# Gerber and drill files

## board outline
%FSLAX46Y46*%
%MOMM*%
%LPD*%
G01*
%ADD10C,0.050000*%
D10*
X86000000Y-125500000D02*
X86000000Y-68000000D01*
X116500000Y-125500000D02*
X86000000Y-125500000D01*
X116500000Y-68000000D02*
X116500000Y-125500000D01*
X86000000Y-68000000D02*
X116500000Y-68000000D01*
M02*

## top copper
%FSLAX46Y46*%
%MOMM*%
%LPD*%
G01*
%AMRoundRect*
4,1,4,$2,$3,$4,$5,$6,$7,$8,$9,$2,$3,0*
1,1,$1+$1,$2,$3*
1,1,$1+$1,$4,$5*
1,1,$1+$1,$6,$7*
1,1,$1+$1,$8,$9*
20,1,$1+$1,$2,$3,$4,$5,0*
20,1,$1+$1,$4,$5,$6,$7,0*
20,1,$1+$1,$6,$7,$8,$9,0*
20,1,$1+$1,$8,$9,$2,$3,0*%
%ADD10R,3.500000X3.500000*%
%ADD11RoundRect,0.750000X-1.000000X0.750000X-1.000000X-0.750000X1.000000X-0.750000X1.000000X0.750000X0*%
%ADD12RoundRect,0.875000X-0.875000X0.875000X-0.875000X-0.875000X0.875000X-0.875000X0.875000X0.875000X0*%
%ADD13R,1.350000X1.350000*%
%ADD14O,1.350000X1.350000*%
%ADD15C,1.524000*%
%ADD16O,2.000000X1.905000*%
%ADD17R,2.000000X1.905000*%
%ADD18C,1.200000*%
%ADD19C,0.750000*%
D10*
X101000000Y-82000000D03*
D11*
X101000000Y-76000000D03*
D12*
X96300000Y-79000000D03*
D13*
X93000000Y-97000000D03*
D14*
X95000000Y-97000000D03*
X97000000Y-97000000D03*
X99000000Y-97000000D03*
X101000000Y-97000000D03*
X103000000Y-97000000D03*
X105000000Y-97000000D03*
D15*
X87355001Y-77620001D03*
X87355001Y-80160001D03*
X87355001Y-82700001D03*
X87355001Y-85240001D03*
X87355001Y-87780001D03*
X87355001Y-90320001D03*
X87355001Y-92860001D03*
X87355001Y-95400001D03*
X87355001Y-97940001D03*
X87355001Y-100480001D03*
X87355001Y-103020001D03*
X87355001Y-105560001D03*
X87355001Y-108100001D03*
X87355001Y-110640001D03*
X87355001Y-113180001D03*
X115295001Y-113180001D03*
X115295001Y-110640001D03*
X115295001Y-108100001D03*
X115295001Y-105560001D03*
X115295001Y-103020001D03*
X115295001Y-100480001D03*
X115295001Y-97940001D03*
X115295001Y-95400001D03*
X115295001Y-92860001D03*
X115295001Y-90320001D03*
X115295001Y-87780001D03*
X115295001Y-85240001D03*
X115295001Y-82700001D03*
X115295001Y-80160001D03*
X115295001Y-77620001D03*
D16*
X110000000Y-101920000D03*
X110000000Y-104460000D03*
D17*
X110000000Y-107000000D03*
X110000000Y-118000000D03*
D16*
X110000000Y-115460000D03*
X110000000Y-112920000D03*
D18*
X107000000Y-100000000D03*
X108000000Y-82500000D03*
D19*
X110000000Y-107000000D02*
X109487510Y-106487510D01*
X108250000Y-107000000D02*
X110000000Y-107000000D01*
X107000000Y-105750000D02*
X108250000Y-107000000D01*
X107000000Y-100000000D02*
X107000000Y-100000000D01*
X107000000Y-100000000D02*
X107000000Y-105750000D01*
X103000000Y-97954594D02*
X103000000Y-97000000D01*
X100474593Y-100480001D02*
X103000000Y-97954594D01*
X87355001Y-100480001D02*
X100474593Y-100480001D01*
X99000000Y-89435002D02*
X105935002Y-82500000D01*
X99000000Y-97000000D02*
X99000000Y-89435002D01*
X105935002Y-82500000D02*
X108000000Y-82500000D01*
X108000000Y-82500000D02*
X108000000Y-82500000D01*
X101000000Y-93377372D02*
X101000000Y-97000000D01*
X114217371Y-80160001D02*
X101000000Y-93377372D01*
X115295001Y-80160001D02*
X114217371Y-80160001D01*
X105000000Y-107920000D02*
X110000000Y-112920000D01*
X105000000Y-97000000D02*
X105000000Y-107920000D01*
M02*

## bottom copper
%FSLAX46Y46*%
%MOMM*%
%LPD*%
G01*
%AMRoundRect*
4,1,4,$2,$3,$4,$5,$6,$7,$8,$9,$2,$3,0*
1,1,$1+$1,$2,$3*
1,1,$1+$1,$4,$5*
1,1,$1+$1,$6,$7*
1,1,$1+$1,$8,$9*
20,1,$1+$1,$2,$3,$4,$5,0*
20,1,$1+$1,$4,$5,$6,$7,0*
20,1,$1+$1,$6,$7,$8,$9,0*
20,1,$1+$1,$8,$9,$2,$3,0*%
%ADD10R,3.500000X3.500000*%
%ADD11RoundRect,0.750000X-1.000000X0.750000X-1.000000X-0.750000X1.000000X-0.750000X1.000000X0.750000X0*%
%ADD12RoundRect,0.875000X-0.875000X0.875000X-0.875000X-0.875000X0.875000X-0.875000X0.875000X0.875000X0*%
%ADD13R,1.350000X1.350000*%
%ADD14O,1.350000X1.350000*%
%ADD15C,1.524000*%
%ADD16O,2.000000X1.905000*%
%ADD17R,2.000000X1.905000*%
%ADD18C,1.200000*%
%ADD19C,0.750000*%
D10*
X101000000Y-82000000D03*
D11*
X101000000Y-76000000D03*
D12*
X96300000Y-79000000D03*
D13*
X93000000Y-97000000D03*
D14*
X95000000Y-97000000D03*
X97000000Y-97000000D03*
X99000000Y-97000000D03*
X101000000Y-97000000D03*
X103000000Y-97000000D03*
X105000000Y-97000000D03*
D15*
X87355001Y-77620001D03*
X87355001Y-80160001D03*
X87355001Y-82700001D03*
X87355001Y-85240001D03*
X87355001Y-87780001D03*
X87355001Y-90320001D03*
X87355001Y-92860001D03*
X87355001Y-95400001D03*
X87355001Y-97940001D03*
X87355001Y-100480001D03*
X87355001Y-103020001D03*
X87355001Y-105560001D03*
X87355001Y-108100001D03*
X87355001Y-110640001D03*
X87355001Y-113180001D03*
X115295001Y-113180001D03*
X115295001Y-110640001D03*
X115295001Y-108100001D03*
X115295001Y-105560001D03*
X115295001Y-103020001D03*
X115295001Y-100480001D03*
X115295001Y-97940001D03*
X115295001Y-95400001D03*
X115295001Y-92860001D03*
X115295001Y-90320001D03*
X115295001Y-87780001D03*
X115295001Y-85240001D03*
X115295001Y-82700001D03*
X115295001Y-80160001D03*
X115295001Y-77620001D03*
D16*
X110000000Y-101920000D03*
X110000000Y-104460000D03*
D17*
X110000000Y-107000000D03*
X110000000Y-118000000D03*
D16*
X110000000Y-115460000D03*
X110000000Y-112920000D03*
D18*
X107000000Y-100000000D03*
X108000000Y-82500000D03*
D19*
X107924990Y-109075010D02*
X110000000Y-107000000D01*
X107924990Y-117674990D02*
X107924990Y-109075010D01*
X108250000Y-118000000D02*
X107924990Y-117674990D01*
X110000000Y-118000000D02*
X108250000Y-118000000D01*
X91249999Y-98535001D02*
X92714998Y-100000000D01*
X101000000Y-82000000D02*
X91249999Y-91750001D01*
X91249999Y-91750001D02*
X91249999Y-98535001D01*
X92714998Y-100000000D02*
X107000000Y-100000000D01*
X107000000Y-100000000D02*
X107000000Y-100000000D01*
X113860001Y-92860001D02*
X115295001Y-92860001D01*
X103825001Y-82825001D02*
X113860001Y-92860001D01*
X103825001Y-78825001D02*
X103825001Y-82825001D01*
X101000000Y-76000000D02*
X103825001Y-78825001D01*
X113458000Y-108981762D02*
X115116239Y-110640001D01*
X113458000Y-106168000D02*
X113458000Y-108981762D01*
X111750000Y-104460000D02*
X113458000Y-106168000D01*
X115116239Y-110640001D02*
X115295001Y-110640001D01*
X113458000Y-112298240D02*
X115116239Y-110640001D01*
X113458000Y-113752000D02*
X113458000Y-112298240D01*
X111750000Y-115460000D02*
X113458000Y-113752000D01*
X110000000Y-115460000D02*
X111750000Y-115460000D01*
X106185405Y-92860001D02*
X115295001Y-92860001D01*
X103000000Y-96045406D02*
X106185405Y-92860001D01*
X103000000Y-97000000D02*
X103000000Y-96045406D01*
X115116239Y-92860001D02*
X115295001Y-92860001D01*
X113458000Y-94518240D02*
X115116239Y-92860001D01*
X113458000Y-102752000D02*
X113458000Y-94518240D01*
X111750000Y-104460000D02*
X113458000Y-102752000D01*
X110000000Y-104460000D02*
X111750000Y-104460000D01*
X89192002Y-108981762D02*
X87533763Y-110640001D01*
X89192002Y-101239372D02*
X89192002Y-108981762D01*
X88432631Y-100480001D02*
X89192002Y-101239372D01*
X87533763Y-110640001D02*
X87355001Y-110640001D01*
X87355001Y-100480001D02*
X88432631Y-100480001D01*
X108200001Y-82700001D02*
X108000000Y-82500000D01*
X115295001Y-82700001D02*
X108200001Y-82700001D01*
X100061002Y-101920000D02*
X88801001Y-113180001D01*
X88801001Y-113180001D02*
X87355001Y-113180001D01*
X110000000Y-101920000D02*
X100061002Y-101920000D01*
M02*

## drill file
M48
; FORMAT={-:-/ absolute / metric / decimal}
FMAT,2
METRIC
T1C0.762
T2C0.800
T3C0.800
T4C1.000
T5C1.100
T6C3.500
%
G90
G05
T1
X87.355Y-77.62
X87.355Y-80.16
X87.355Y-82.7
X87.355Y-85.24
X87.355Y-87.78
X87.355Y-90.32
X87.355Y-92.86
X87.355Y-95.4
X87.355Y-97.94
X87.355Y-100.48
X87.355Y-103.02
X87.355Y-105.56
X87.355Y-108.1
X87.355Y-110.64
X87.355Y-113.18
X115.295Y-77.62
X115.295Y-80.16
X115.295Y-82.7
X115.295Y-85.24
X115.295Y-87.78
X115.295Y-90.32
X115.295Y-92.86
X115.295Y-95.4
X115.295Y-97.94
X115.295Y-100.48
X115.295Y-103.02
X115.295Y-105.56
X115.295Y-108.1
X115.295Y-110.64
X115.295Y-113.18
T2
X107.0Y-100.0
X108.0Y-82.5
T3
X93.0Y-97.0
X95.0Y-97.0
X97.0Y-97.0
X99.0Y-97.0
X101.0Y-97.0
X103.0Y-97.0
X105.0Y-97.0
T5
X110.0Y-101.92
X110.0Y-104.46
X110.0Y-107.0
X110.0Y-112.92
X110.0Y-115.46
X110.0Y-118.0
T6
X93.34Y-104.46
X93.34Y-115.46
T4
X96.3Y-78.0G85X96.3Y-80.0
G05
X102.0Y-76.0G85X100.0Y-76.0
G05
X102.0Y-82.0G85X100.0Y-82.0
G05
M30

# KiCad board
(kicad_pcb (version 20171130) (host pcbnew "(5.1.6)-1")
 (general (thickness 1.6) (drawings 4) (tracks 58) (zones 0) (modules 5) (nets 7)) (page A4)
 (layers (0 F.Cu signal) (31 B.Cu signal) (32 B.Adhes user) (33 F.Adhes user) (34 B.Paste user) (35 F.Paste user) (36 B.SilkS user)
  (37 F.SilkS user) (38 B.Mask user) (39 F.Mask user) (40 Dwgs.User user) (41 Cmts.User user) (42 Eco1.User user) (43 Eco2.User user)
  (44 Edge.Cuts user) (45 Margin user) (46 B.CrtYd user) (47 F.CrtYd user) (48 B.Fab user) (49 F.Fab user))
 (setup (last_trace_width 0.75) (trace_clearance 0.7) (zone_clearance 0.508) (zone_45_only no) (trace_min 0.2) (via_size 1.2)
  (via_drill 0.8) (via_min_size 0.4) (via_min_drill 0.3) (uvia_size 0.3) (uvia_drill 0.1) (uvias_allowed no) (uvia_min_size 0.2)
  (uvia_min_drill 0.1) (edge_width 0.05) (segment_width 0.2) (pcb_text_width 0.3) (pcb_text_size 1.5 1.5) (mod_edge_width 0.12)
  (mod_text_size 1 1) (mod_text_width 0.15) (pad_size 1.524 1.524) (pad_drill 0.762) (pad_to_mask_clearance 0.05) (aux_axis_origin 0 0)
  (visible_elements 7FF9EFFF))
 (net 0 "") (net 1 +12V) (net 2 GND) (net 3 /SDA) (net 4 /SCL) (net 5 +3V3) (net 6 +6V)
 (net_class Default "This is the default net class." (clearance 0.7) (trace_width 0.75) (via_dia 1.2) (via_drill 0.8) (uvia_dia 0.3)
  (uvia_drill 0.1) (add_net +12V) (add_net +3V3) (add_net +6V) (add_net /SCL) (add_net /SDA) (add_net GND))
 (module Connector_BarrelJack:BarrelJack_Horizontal (layer F.Cu) (at 101 82 270)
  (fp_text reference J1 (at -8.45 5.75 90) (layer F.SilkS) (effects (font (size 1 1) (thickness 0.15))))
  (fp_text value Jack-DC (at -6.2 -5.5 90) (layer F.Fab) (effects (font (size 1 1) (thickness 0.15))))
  (pad 1 thru_hole rect (at 0 0 270) (size 3.5 3.5) (drill oval 1 3) (layers *.Cu *.Mask) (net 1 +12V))
  (pad 2 thru_hole roundrect (at -6 0 270) (size 3 3.5) (drill oval 1 3) (layers *.Cu *.Mask) (roundrect_rratio 0.25) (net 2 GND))
  (pad 3 thru_hole roundrect (at -3 4.7 270) (size 3.5 3.5) (drill oval 3 1) (layers *.Cu *.Mask) (roundrect_rratio 0.25)))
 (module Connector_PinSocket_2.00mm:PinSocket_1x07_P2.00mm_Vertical (layer F.Cu) (at 93 97 90)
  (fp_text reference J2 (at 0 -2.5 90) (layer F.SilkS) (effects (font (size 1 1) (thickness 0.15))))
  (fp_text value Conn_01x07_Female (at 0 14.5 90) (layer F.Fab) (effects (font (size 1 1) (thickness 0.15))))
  (pad 1 thru_hole rect (at 0 0 90) (size 1.35 1.35) (drill 0.8) (layers *.Cu *.Mask))
  (pad 2 thru_hole oval (at 0 2 90) (size 1.35 1.35) (drill 0.8) (layers *.Cu *.Mask))
  (pad 3 thru_hole oval (at 0 4 90) (size 1.35 1.35) (drill 0.8) (layers *.Cu *.Mask))
  (pad 4 thru_hole oval (at 0 6 90) (size 1.35 1.35) (drill 0.8) (layers *.Cu *.Mask) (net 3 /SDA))
  (pad 5 thru_hole oval (at 0 8 90) (size 1.35 1.35) (drill 0.8) (layers *.Cu *.Mask) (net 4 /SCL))
  (pad 6 thru_hole oval (at 0 10 90) (size 1.35 1.35) (drill 0.8) (layers *.Cu *.Mask) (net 2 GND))
  (pad 7 thru_hole oval (at 0 12 90) (size 1.35 1.35) (drill 0.8) (layers *.Cu *.Mask) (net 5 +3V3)))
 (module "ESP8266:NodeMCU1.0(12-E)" (layer F.Cu) (at 101.325001 98.575001)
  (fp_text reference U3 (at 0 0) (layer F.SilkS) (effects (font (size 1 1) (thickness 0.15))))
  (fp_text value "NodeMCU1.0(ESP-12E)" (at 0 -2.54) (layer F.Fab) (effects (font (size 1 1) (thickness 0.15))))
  (pad 1 thru_hole circle (at -13.97 -20.955) (size 1.524 1.524) (drill 0.762) (layers *.Cu *.Mask F.SilkS))
  (pad 2 thru_hole circle (at -13.97 -18.415) (size 1.524 1.524) (drill 0.762) (layers *.Cu *.Mask F.SilkS))
  (pad 3 thru_hole circle (at -13.97 -15.875) (size 1.524 1.524) (drill 0.762) (layers *.Cu *.Mask F.SilkS))
  (pad 4 thru_hole circle (at -13.97 -13.335) (size 1.524 1.524) (drill 0.762) (layers *.Cu *.Mask F.SilkS))
  (pad 5 thru_hole circle (at -13.97 -10.795) (size 1.524 1.524) (drill 0.762) (layers *.Cu *.Mask F.SilkS))
  (pad 6 thru_hole circle (at -13.97 -8.255) (size 1.524 1.524) (drill 0.762) (layers *.Cu *.Mask F.SilkS))
  (pad 7 thru_hole circle (at -13.97 -5.715) (size 1.524 1.524) (drill 0.762) (layers *.Cu *.Mask F.SilkS))
  (pad 8 thru_hole circle (at -13.97 -3.175) (size 1.524 1.524) (drill 0.762) (layers *.Cu *.Mask F.SilkS))
  (pad 9 thru_hole circle (at -13.97 -0.635) (size 1.524 1.524) (drill 0.762) (layers *.Cu *.Mask F.SilkS))
  (pad 10 thru_hole circle (at -13.97 1.905) (size 1.524 1.524) (drill 0.762) (layers *.Cu *.Mask F.SilkS) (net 2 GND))
  (pad 11 thru_hole circle (at -13.97 4.445) (size 1.524 1.524) (drill 0.762) (layers *.Cu *.Mask F.SilkS))
  (pad 12 thru_hole circle (at -13.97 6.985) (size 1.524 1.524) (drill 0.762) (layers *.Cu *.Mask F.SilkS))
  (pad 13 thru_hole circle (at -13.97 9.525) (size 1.524 1.524) (drill 0.762) (layers *.Cu *.Mask F.SilkS))
  (pad 14 thru_hole circle (at -13.97 12.065) (size 1.524 1.524) (drill 0.762) (layers *.Cu *.Mask F.SilkS) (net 2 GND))
  (pad 15 thru_hole circle (at -13.97 14.605) (size 1.524 1.524) (drill 0.762) (layers *.Cu *.Mask F.SilkS) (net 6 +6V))
  (pad 16 thru_hole circle (at 13.97 14.605) (size 1.524 1.524) (drill 0.762) (layers *.Cu *.Mask F.SilkS))
  (pad 17 thru_hole circle (at 13.97 12.065) (size 1.524 1.524) (drill 0.762) (layers *.Cu *.Mask F.SilkS) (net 2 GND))
  (pad 18 thru_hole circle (at 13.97 9.525) (size 1.524 1.524) (drill 0.762) (layers *.Cu *.Mask F.SilkS))
  (pad 19 thru_hole circle (at 13.97 6.985) (size 1.524 1.524) (drill 0.762) (layers *.Cu *.Mask F.SilkS))
  (pad 20 thru_hole circle (at 13.97 4.445) (size 1.524 1.524) (drill 0.762) (layers *.Cu *.Mask F.SilkS))
  (pad 21 thru_hole circle (at 13.97 1.905) (size 1.524 1.524) (drill 0.762) (layers *.Cu *.Mask F.SilkS))
  (pad 22 thru_hole circle (at 13.97 -0.635) (size 1.524 1.524) (drill 0.762) (layers *.Cu *.Mask F.SilkS))
  (pad 23 thru_hole circle (at 13.97 -3.175) (size 1.524 1.524) (drill 0.762) (layers *.Cu *.Mask F.SilkS))
  (pad 24 thru_hole circle (at 13.97 -5.715) (size 1.524 1.524) (drill 0.762) (layers *.Cu *.Mask F.SilkS) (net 2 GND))
  (pad 25 thru_hole circle (at 13.97 -8.255) (size 1.524 1.524) (drill 0.762) (layers *.Cu *.Mask F.SilkS))
  (pad 26 thru_hole circle (at 13.97 -10.795) (size 1.524 1.524) (drill 0.762) (layers *.Cu *.Mask F.SilkS))
  (pad 27 thru_hole circle (at 13.97 -13.335) (size 1.524 1.524) (drill 0.762) (layers *.Cu *.Mask F.SilkS))
  (pad 28 thru_hole circle (at 13.97 -15.875) (size 1.524 1.524) (drill 0.762) (layers *.Cu *.Mask F.SilkS) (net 3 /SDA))
  (pad 29 thru_hole circle (at 13.97 -18.415) (size 1.524 1.524) (drill 0.762) (layers *.Cu *.Mask F.SilkS) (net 4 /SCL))
  (pad 30 thru_hole circle (at 13.97 -20.955) (size 1.524 1.524) (drill 0.762) (layers *.Cu *.Mask F.SilkS)))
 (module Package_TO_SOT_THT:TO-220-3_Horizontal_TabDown (layer F.Cu) (at 110 107 90)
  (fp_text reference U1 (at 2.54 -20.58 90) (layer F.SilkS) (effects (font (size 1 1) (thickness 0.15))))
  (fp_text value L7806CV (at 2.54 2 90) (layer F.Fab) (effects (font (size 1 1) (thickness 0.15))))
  (pad 3 thru_hole oval (at 5.08 0 90) (size 1.905 2) (drill 1.1) (layers *.Cu *.Mask) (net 6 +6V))
  (pad 2 thru_hole oval (at 2.54 0 90) (size 1.905 2) (drill 1.1) (layers *.Cu *.Mask) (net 2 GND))
  (pad 1 thru_hole rect (at 0 0 90) (size 1.905 2) (drill 1.1) (layers *.Cu *.Mask) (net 1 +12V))
  (pad "" np_thru_hole oval (at 2.54 -16.66 90) (size 3.5 3.5) (drill 3.5) (layers *.Cu *.Mask)))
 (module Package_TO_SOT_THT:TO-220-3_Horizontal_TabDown (layer F.Cu) (at 110 118 90)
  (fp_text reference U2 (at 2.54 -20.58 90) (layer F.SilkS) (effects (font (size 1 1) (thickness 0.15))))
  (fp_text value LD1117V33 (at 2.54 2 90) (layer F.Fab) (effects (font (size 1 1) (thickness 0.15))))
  (pad "" np_thru_hole oval (at 2.54 -16.66 90) (size 3.5 3.5) (drill 3.5) (layers *.Cu *.Mask))
  (pad 1 thru_hole rect (at 0 0 90) (size 1.905 2) (drill 1.1) (layers *.Cu *.Mask) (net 1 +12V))
  (pad 2 thru_hole oval (at 2.54 0 90) (size 1.905 2) (drill 1.1) (layers *.Cu *.Mask) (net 2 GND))
  (pad 3 thru_hole oval (at 5.08 0 90) (size 1.905 2) (drill 1.1) (layers *.Cu *.Mask) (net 5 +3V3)))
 (gr_line (start 86 125.5) (end 86 68) (layer Edge.Cuts) (width 0.05))
 (gr_line (start 116.5 125.5) (end 86 125.5) (layer Edge.Cuts) (width 0.05))
 (gr_line (start 116.5 68) (end 116.5 125.5) (layer Edge.Cuts) (width 0.05))
 (gr_line (start 86 68) (end 116.5 68) (layer Edge.Cuts) (width 0.05))
 (segment (start 107.92499 109.07501) (end 110 107) (width 0.75) (layer B.Cu) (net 1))
 (segment (start 107.92499 117.67499) (end 107.92499 109.07501) (width 0.75) (layer B.Cu) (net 1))
 (segment (start 108.25 118) (end 107.92499 117.67499) (width 0.75) (layer B.Cu) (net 1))
 (segment (start 110 118) (end 108.25 118) (width 0.75) (layer B.Cu) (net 1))
 (segment (start 110 107) (end 109.48751 106.48751) (width 0.75) (layer F.Cu) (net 1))
 (segment (start 91.249999 98.535001) (end 92.714998 100) (width 0.75) (layer B.Cu) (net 1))
 (segment (start 101 82) (end 91.249999 91.750001) (width 0.75) (layer B.Cu) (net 1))
 (segment (start 91.249999 91.750001) (end 91.249999 98.535001) (width 0.75) (layer B.Cu) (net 1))
 (segment (start 92.714998 100) (end 107 100) (width 0.75) (layer B.Cu) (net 1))
 (segment (start 107 100) (end 107 100) (width 0.75) (layer B.Cu) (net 1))
 (segment (start 108.25 107) (end 110 107) (width 0.75) (layer F.Cu) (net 1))
 (segment (start 107 105.75) (end 108.25 107) (width 0.75) (layer F.Cu) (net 1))
 (segment (start 107 100) (end 107 100) (width 0.75) (layer F.Cu) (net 1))
 (segment (start 107 100) (end 107 105.75) (width 0.75) (layer F.Cu) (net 1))
 (via (at 107 100) (size 1.2) (drill 0.8) (layers F.Cu B.Cu) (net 1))
 (segment (start 113.860001 92.860001) (end 115.295001 92.860001) (width 0.75) (layer B.Cu) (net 2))
 (segment (start 103.825001 82.825001) (end 113.860001 92.860001) (width 0.75) (layer B.Cu) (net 2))
 (segment (start 103.825001 78.825001) (end 103.825001 82.825001) (width 0.75) (layer B.Cu) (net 2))
 (segment (start 101 76) (end 103.825001 78.825001) (width 0.75) (layer B.Cu) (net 2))
 (segment (start 113.458 108.981762) (end 115.116239 110.640001) (width 0.75) (layer B.Cu) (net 2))
 (segment (start 113.458 106.168) (end 113.458 108.981762) (width 0.75) (layer B.Cu) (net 2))
 (segment (start 111.75 104.46) (end 113.458 106.168) (width 0.75) (layer B.Cu) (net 2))
 (segment (start 115.116239 110.640001) (end 115.295001 110.640001) (width 0.75) (layer B.Cu) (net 2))
 (segment (start 113.458 112.29824) (end 115.116239 110.640001) (width 0.75) (layer B.Cu) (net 2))
 (segment (start 113.458 113.752) (end 113.458 112.29824) (width 0.75) (layer B.Cu) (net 2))
 (segment (start 111.75 115.46) (end 113.458 113.752) (width 0.75) (layer B.Cu) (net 2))
 (segment (start 110 115.46) (end 111.75 115.46) (width 0.75) (layer B.Cu) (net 2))
 (segment (start 106.185405 92.860001) (end 115.295001 92.860001) (width 0.75) (layer B.Cu) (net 2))
 (segment (start 103 96.045406) (end 106.185405 92.860001) (width 0.75) (layer B.Cu) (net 2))
 (segment (start 103 97) (end 103 96.045406) (width 0.75) (layer B.Cu) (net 2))
 (segment (start 115.116239 92.860001) (end 115.295001 92.860001) (width 0.75) (layer B.Cu) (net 2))
 (segment (start 113.458 94.51824) (end 115.116239 92.860001) (width 0.75) (layer B.Cu) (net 2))
 (segment (start 113.458 102.752) (end 113.458 94.51824) (width 0.75) (layer B.Cu) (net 2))
 (segment (start 111.75 104.46) (end 113.458 102.752) (width 0.75) (layer B.Cu) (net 2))
 (segment (start 110 104.46) (end 111.75 104.46) (width 0.75) (layer B.Cu) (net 2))
 (segment (start 89.192002 108.981762) (end 87.533763 110.640001) (width 0.75) (layer B.Cu) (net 2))
 (segment (start 89.192002 101.239372) (end 89.192002 108.981762) (width 0.75) (layer B.Cu) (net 2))
 (segment (start 88.432631 100.480001) (end 89.192002 101.239372) (width 0.75) (layer B.Cu) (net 2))
 (segment (start 87.533763 110.640001) (end 87.355001 110.640001) (width 0.75) (layer B.Cu) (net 2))
 (segment (start 87.355001 100.480001) (end 88.432631 100.480001) (width 0.75) (layer B.Cu) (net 2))
 (segment (start 103 97.954594) (end 103 97) (width 0.75) (layer F.Cu) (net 2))
 (segment (start 100.474593 100.480001) (end 103 97.954594) (width 0.75) (layer F.Cu) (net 2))
 (segment (start 87.355001 100.480001) (end 100.474593 100.480001) (width 0.75) (layer F.Cu) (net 2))
 (segment (start 99 89.435002) (end 105.935002 82.5) (width 0.75) (layer F.Cu) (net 3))
 (segment (start 99 97) (end 99 89.435002) (width 0.75) (layer F.Cu) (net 3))
 (segment (start 105.935002 82.5) (end 108 82.5) (width 0.75) (layer F.Cu) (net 3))
 (segment (start 108 82.5) (end 108 82.5) (width 0.75) (layer F.Cu) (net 3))
 (via (at 108 82.5) (size 1.2) (drill 0.8) (layers F.Cu B.Cu) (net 3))
 (segment (start 108.200001 82.700001) (end 108 82.5) (width 0.75) (layer B.Cu) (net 3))
 (segment (start 115.295001 82.700001) (end 108.200001 82.700001) (width 0.75) (layer B.Cu) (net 3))
 (segment (start 101 93.377372) (end 101 97) (width 0.75) (layer F.Cu) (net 4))
 (segment (start 114.217371 80.160001) (end 101 93.377372) (width 0.75) (layer F.Cu) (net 4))
 (segment (start 115.295001 80.160001) (end 114.217371 80.160001) (width 0.75) (layer F.Cu) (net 4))
 (segment (start 105 107.92) (end 110 112.92) (width 0.75) (layer F.Cu) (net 5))
 (segment (start 105 97) (end 105 107.92) (width 0.75) (layer F.Cu) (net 5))
 (segment (start 100.061002 101.92) (end 88.801001 113.180001) (width 0.75) (layer B.Cu) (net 6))
 (segment (start 88.801001 113.180001) (end 87.355001 113.180001) (width 0.75) (layer B.Cu) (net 6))
 (segment (start 110 101.92) (end 100.061002 101.92) (width 0.75) (layer B.Cu) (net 6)))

